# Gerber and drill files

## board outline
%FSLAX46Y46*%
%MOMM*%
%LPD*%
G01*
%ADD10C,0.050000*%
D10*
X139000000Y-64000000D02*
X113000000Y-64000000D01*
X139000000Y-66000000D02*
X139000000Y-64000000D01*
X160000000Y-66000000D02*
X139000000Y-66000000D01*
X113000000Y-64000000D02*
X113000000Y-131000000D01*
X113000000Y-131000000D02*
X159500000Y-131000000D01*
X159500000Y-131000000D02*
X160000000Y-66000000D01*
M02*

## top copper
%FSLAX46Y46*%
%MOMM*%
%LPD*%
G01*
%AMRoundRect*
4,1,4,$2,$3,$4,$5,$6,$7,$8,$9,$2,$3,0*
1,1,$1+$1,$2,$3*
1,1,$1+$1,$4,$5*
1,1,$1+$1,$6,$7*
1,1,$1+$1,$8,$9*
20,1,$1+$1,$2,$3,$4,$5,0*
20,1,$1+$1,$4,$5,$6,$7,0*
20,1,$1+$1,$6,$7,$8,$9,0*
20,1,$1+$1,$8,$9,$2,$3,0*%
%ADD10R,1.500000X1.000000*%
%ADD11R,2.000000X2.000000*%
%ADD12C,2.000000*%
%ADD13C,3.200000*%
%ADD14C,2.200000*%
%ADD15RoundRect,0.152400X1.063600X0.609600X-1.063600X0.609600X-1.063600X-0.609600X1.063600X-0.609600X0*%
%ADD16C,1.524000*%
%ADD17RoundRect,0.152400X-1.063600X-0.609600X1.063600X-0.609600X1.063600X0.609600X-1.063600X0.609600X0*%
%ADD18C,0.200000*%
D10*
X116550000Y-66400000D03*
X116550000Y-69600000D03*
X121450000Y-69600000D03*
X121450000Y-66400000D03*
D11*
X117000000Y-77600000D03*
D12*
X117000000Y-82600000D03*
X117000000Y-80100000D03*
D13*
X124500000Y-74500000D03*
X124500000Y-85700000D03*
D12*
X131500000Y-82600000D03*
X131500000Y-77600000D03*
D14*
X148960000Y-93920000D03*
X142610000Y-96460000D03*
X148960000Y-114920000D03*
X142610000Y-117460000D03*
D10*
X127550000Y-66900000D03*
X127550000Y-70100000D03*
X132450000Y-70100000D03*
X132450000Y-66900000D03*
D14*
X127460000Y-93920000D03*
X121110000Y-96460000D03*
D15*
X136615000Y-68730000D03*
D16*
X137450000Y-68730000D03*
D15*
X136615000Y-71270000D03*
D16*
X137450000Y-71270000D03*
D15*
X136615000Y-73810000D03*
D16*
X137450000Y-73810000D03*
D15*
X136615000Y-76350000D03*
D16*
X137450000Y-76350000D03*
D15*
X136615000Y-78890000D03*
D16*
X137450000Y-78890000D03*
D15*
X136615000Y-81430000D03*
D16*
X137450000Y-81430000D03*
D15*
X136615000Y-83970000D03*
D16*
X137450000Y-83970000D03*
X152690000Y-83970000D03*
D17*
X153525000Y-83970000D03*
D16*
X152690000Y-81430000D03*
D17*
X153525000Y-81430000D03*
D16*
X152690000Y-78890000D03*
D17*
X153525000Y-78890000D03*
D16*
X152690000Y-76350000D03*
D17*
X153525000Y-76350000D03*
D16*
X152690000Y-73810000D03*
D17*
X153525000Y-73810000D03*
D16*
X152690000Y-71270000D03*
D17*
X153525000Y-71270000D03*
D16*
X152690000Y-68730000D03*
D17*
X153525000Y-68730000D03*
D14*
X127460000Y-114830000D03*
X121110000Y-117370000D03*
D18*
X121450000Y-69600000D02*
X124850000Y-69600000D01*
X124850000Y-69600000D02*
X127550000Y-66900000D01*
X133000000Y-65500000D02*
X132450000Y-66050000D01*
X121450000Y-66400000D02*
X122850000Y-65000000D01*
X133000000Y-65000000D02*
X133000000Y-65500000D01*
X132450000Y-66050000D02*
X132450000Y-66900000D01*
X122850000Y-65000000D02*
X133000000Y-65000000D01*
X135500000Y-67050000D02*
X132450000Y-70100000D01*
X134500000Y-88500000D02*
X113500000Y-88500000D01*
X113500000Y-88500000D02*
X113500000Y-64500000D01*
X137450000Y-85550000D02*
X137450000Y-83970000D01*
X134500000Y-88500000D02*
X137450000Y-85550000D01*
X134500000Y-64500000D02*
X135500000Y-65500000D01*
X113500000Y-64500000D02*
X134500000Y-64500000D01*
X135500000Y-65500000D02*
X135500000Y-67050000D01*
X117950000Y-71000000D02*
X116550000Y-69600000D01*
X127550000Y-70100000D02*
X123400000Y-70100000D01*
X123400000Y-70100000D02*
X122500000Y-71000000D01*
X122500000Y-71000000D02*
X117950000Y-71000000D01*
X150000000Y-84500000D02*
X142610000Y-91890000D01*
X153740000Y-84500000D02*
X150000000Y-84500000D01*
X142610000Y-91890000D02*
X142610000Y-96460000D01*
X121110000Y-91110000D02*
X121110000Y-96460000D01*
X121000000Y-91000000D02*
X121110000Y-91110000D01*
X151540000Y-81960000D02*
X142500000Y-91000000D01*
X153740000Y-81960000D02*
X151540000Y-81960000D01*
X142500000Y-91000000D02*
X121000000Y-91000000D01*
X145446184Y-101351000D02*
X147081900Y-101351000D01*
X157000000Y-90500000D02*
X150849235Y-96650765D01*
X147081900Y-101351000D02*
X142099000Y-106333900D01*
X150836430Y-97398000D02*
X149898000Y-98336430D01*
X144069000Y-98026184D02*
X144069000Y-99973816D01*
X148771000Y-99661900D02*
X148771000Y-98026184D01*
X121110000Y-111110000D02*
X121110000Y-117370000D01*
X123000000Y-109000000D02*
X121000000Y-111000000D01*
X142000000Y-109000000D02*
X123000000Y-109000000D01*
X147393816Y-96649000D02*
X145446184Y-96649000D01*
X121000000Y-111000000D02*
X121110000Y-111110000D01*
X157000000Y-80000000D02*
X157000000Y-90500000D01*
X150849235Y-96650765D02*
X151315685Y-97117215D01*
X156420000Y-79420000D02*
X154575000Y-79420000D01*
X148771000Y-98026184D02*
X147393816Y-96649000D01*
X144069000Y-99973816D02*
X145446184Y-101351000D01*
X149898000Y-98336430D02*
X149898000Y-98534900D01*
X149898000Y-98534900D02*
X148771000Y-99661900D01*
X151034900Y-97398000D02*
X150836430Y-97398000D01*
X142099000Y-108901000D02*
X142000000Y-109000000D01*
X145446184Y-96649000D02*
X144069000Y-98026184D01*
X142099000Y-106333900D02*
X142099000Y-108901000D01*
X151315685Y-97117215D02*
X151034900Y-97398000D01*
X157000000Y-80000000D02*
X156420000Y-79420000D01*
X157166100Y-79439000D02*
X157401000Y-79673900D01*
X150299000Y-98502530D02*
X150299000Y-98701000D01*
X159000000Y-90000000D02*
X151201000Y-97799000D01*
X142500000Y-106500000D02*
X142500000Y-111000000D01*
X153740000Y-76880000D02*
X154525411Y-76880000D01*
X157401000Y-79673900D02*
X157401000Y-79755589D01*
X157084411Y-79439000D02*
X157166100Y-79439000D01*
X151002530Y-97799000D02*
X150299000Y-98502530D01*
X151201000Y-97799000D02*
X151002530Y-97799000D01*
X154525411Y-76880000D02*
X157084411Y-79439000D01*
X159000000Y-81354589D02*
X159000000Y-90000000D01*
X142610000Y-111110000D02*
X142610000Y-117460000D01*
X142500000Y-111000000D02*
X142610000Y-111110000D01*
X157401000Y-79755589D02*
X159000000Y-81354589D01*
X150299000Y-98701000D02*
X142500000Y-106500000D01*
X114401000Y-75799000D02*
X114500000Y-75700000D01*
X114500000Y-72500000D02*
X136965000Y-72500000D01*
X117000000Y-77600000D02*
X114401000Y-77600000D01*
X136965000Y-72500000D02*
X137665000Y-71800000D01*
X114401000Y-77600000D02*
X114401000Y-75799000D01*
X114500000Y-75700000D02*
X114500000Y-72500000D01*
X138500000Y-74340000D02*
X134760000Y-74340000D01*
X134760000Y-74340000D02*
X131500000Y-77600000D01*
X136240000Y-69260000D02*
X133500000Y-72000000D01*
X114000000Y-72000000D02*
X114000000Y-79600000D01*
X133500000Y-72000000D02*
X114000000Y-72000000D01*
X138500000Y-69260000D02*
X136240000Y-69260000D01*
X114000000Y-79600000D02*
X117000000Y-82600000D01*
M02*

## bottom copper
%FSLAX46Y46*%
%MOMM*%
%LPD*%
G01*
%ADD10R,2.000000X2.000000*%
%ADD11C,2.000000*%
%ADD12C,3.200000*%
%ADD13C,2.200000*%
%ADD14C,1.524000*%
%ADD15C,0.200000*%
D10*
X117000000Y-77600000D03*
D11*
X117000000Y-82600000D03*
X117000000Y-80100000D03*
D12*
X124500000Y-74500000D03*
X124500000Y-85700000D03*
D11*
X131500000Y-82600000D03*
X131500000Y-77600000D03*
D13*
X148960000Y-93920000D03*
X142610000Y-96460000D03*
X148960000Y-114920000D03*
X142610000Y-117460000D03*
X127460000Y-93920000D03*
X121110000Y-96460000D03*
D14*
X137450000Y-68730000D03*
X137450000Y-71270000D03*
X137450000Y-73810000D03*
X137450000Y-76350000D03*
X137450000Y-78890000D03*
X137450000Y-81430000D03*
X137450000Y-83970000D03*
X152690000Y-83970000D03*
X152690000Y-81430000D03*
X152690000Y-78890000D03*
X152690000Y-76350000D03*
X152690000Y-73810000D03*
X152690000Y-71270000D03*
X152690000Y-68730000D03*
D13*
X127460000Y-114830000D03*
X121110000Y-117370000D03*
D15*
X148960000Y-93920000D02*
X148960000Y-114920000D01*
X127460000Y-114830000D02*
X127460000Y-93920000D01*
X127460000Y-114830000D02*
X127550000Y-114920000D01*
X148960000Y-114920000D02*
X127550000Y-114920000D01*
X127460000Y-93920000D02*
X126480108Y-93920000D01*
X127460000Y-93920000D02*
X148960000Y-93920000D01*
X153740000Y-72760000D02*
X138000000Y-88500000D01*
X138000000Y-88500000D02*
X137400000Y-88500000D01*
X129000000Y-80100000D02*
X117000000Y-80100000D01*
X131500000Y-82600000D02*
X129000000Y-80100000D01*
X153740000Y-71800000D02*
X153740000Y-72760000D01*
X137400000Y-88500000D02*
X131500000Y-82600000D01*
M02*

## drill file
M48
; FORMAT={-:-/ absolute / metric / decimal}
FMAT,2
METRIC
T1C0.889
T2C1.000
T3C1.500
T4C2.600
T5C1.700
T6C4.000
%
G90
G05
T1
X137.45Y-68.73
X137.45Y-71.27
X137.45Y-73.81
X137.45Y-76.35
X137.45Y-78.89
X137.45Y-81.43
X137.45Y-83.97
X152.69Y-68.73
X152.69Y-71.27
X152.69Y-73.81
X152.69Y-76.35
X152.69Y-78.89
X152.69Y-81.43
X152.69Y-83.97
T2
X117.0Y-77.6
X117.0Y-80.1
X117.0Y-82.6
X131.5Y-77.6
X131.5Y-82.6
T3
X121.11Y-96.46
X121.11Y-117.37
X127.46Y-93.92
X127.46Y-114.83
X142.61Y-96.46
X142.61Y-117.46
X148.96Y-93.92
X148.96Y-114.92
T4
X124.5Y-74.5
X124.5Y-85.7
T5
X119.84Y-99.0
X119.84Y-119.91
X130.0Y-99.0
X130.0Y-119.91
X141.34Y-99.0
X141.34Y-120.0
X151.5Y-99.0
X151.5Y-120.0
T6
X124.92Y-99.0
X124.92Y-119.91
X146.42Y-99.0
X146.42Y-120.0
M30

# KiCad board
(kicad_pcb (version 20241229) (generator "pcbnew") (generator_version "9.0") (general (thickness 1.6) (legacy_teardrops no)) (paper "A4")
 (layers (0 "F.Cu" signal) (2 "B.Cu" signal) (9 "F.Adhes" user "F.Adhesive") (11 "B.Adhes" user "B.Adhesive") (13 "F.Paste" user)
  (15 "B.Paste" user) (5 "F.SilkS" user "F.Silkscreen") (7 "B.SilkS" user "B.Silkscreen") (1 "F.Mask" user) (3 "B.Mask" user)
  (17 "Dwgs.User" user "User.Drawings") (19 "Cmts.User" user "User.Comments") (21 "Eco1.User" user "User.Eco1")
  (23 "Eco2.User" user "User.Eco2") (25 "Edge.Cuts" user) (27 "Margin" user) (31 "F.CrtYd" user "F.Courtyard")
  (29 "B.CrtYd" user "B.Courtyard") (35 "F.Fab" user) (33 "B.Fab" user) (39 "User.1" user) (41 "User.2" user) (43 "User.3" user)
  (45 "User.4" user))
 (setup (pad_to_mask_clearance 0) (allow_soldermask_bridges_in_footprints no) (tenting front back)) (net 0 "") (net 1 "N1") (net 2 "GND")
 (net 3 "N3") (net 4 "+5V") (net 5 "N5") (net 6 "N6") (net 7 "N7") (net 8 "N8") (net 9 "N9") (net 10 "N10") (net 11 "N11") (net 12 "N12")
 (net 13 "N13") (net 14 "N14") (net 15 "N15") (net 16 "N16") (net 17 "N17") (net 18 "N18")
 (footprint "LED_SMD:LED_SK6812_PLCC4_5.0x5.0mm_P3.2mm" (layer "F.Cu") (at 119 68)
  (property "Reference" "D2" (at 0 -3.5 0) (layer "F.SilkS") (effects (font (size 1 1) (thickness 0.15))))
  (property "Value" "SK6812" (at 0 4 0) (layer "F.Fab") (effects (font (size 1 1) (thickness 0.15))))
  (pad "1" smd rect (at -2.45 -1.6 180) (size 1.5 1) (layers "F.Cu" "F.Mask" "F.Paste") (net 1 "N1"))
  (pad "2" smd rect (at -2.45 1.6 180) (size 1.5 1) (layers "F.Cu" "F.Mask" "F.Paste") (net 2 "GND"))
  (pad "3" smd rect (at 2.45 1.6 180) (size 1.5 1) (layers "F.Cu" "F.Mask" "F.Paste") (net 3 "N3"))
  (pad "4" smd rect (at 2.45 -1.6 180) (size 1.5 1) (layers "F.Cu" "F.Mask" "F.Paste") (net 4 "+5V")))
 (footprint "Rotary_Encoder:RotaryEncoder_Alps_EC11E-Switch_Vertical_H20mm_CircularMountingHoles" (layer "F.Cu") (at 117 77.6)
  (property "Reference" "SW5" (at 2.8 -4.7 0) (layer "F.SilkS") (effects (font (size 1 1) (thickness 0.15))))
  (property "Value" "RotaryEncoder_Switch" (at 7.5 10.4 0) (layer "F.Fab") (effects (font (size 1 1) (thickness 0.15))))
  (pad "A" thru_hole rect (at 0 0) (size 2 2) (drill 1) (layers "*.Cu" "*.Mask") (remove_unused_layers no) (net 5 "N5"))
  (pad "B" thru_hole circle (at 0 5) (size 2 2) (drill 1) (layers "*.Cu" "*.Mask") (remove_unused_layers no) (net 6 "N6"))
  (pad "C" thru_hole circle (at 0 2.5) (size 2 2) (drill 1) (layers "*.Cu" "*.Mask") (remove_unused_layers no) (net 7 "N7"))
  (pad "MP" thru_hole circle (at 7.5 -3.1) (size 3.2 3.2) (drill 2.6) (layers "*.Cu" "*.Mask") (remove_unused_layers no))
  (pad "MP" thru_hole circle (at 7.5 8.1) (size 3.2 3.2) (drill 2.6) (layers "*.Cu" "*.Mask") (remove_unused_layers no))
  (pad "S1" thru_hole circle (at 14.5 5) (size 2 2) (drill 1) (layers "*.Cu" "*.Mask") (remove_unused_layers no) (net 7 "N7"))
  (pad "S2" thru_hole circle (at 14.5 0) (size 2 2) (drill 1) (layers "*.Cu" "*.Mask") (remove_unused_layers no) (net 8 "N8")))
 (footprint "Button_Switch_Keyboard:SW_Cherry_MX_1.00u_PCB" (layer "F.Cu") (at 148.96 93.92)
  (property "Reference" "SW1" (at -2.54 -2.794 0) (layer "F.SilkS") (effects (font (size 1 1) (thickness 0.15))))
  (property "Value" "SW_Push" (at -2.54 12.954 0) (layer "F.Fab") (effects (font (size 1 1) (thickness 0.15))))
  (pad "" np_thru_hole circle (at -7.62 5.08) (size 1.7 1.7) (drill 1.7) (layers "*.Cu" "*.Mask"))
  (pad "" np_thru_hole circle (at -2.54 5.08) (size 4 4) (drill 4) (layers "*.Cu" "*.Mask"))
  (pad "" np_thru_hole circle (at 2.54 5.08) (size 1.7 1.7) (drill 1.7) (layers "*.Cu" "*.Mask"))
  (pad "1" thru_hole circle (at 0 0) (size 2.2 2.2) (drill 1.5) (layers "*.Cu" "*.Mask") (remove_unused_layers no) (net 2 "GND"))
  (pad "2" thru_hole circle (at -6.35 2.54) (size 2.2 2.2) (drill 1.5) (layers "*.Cu" "*.Mask") (remove_unused_layers no) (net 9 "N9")))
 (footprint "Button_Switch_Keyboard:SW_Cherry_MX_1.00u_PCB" (layer "F.Cu") (at 148.96 114.92)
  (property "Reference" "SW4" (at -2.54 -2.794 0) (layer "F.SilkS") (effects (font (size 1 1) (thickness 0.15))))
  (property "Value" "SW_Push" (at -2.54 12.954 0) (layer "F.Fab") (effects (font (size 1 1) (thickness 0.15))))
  (pad "" np_thru_hole circle (at -7.62 5.08) (size 1.7 1.7) (drill 1.7) (layers "*.Cu" "*.Mask"))
  (pad "" np_thru_hole circle (at -2.54 5.08) (size 4 4) (drill 4) (layers "*.Cu" "*.Mask"))
  (pad "" np_thru_hole circle (at 2.54 5.08) (size 1.7 1.7) (drill 1.7) (layers "*.Cu" "*.Mask"))
  (pad "1" thru_hole circle (at 0 0) (size 2.2 2.2) (drill 1.5) (layers "*.Cu" "*.Mask") (remove_unused_layers no) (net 2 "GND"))
  (pad "2" thru_hole circle (at -6.35 2.54) (size 2.2 2.2) (drill 1.5) (layers "*.Cu" "*.Mask") (remove_unused_layers no) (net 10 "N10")))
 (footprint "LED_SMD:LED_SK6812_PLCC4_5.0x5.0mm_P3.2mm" (layer "F.Cu") (at 130 68.5)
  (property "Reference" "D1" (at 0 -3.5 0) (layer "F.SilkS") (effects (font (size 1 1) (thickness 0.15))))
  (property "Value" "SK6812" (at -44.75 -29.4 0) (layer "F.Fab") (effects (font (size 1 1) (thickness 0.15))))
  (pad "1" smd rect (at -2.45 -1.6 180) (size 1.5 1) (layers "F.Cu" "F.Mask" "F.Paste") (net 3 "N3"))
  (pad "2" smd rect (at -2.45 1.6 180) (size 1.5 1) (layers "F.Cu" "F.Mask" "F.Paste") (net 2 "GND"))
  (pad "3" smd rect (at 2.45 1.6 180) (size 1.5 1) (layers "F.Cu" "F.Mask" "F.Paste") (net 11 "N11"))
  (pad "4" smd rect (at 2.45 -1.6 180) (size 1.5 1) (layers "F.Cu" "F.Mask" "F.Paste") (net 4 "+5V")))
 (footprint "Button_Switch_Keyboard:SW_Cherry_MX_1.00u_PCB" (layer "F.Cu") (at 127.46 93.92)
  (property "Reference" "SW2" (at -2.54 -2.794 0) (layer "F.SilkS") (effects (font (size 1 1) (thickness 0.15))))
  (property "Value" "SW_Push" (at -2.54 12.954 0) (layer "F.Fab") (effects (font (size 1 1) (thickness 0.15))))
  (pad "" np_thru_hole circle (at -7.62 5.08) (size 1.7 1.7) (drill 1.7) (layers "*.Cu" "*.Mask"))
  (pad "" np_thru_hole circle (at -2.54 5.08) (size 4 4) (drill 4) (layers "*.Cu" "*.Mask"))
  (pad "" np_thru_hole circle (at 2.54 5.08) (size 1.7 1.7) (drill 1.7) (layers "*.Cu" "*.Mask"))
  (pad "1" thru_hole circle (at 0 0) (size 2.2 2.2) (drill 1.5) (layers "*.Cu" "*.Mask") (remove_unused_layers no) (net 2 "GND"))
  (pad "2" thru_hole circle (at -6.35 2.54) (size 2.2 2.2) (drill 1.5) (layers "*.Cu" "*.Mask") (remove_unused_layers no) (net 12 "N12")))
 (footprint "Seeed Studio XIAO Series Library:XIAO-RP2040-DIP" (layer "F.Cu") (at 145.07 76.35)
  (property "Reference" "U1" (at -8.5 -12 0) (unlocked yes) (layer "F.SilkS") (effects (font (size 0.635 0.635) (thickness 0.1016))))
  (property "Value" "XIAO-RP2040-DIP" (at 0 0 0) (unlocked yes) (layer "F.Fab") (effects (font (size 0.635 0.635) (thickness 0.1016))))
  (pad "1" smd roundrect (at -8.455 -7.62 180) (size 2.432 1.524) (layers "F.Cu" "F.Mask") (roundrect_rratio 0.1) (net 6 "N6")
   (thermal_bridge_angle 45))
  (pad "1" thru_hole circle (at -7.62 -7.62 180) (size 1.524 1.524) (drill 0.889) (layers "*.Cu" "*.Mask") (remove_unused_layers no)
   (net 6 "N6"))
  (pad "2" smd roundrect (at -8.455 -5.08 180) (size 2.432 1.524) (layers "F.Cu" "F.Mask") (roundrect_rratio 0.1) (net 5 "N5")
   (thermal_bridge_angle 45))
  (pad "2" thru_hole circle (at -7.62 -5.08 180) (size 1.524 1.524) (drill 0.889) (layers "*.Cu" "*.Mask") (remove_unused_layers no)
   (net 5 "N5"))
  (pad "3" smd roundrect (at -8.455 -2.54 180) (size 2.432 1.524) (layers "F.Cu" "F.Mask") (roundrect_rratio 0.1) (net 8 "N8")
   (thermal_bridge_angle 45))
  (pad "3" thru_hole circle (at -7.62 -2.54 180) (size 1.524 1.524) (drill 0.889) (layers "*.Cu" "*.Mask") (remove_unused_layers no)
   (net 8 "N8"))
  (pad "4" smd roundrect (at -8.455 0 180) (size 2.432 1.524) (layers "F.Cu" "F.Mask") (roundrect_rratio 0.1) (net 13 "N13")
   (thermal_bridge_angle 45))
  (pad "4" thru_hole circle (at -7.62 0 180) (size 1.524 1.524) (drill 0.889) (layers "*.Cu" "*.Mask") (remove_unused_layers no)
   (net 13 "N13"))
  (pad "5" smd roundrect (at -8.455 2.54 180) (size 2.432 1.524) (layers "F.Cu" "F.Mask") (roundrect_rratio 0.1) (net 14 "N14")
   (thermal_bridge_angle 45))
  (pad "5" thru_hole circle (at -7.62 2.54 180) (size 1.524 1.524) (drill 0.889) (layers "*.Cu" "*.Mask") (remove_unused_layers no)
   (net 14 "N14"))
  (pad "6" smd roundrect (at -8.455 5.08 180) (size 2.432 1.524) (layers "F.Cu" "F.Mask") (roundrect_rratio 0.1) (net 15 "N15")
   (thermal_bridge_angle 45))
  (pad "6" thru_hole circle (at -7.62 5.08 180) (size 1.524 1.524) (drill 0.889) (layers "*.Cu" "*.Mask") (remove_unused_layers no)
   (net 15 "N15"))
  (pad "7" smd roundrect (at -8.455 7.62 180) (size 2.432 1.524) (layers "F.Cu" "F.Mask") (roundrect_rratio 0.1) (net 11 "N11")
   (thermal_bridge_angle 45))
  (pad "7" thru_hole circle (at -7.62 7.62 180) (size 1.524 1.524) (drill 0.889) (layers "*.Cu" "*.Mask") (remove_unused_layers no)
   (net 11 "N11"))
  (pad "8" thru_hole circle (at 7.62 7.62) (size 1.524 1.524) (drill 0.889) (layers "*.Cu" "*.Mask") (remove_unused_layers no) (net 9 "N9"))
  (pad "8" smd roundrect (at 8.455 7.62) (size 2.432 1.524) (layers "F.Cu" "F.Mask") (roundrect_rratio 0.1) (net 9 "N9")
   (thermal_bridge_angle 45))
  (pad "9" thru_hole circle (at 7.62 5.08) (size 1.524 1.524) (drill 0.889) (layers "*.Cu" "*.Mask") (remove_unused_layers no)
   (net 12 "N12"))
  (pad "9" smd roundrect (at 8.455 5.08) (size 2.432 1.524) (layers "F.Cu" "F.Mask") (roundrect_rratio 0.1) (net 12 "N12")
   (thermal_bridge_angle 45))
  (pad "10" thru_hole circle (at 7.62 2.54) (size 1.524 1.524) (drill 0.889) (layers "*.Cu" "*.Mask") (remove_unused_layers no)
   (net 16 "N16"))
  (pad "10" smd roundrect (at 8.455 2.54) (size 2.432 1.524) (layers "F.Cu" "F.Mask") (roundrect_rratio 0.1) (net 16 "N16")
   (thermal_bridge_angle 45))
  (pad "11" thru_hole circle (at 7.62 0) (size 1.524 1.524) (drill 0.889) (layers "*.Cu" "*.Mask") (remove_unused_layers no) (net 10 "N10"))
  (pad "11" smd roundrect (at 8.455 0) (size 2.432 1.524) (layers "F.Cu" "F.Mask") (roundrect_rratio 0.1) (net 10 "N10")
   (thermal_bridge_angle 45))
  (pad "12" thru_hole circle (at 7.62 -2.54) (size 1.524 1.524) (drill 0.889) (layers "*.Cu" "*.Mask") (remove_unused_layers no)
   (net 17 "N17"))
  (pad "12" smd roundrect (at 8.455 -2.54) (size 2.432 1.524) (layers "F.Cu" "F.Mask") (roundrect_rratio 0.1) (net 17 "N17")
   (thermal_bridge_angle 45))
  (pad "13" thru_hole circle (at 7.62 -5.08) (size 1.524 1.524) (drill 0.889) (layers "*.Cu" "*.Mask") (remove_unused_layers no)
   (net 7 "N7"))
  (pad "13" smd roundrect (at 8.455 -5.08) (size 2.432 1.524) (layers "F.Cu" "F.Mask") (roundrect_rratio 0.1) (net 7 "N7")
   (thermal_bridge_angle 45))
  (pad "14" thru_hole circle (at 7.62 -7.62) (size 1.524 1.524) (drill 0.889) (layers "*.Cu" "*.Mask") (remove_unused_layers no)
   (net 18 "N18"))
  (pad "14" smd roundrect (at 8.455 -7.62) (size 2.432 1.524) (layers "F.Cu" "F.Mask") (roundrect_rratio 0.1) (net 18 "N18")
   (thermal_bridge_angle 45)))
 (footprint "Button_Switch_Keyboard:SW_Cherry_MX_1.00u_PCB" (layer "F.Cu") (at 127.46 114.83)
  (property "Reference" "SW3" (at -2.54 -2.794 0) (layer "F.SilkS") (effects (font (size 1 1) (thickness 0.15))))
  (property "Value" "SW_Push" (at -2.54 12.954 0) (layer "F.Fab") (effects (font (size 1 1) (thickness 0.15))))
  (pad "" np_thru_hole circle (at -7.62 5.08) (size 1.7 1.7) (drill 1.7) (layers "*.Cu" "*.Mask"))
  (pad "" np_thru_hole circle (at -2.54 5.08) (size 4 4) (drill 4) (layers "*.Cu" "*.Mask"))
  (pad "" np_thru_hole circle (at 2.54 5.08) (size 1.7 1.7) (drill 1.7) (layers "*.Cu" "*.Mask"))
  (pad "1" thru_hole circle (at 0 0) (size 2.2 2.2) (drill 1.5) (layers "*.Cu" "*.Mask") (remove_unused_layers no) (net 2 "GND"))
  (pad "2" thru_hole circle (at -6.35 2.54) (size 2.2 2.2) (drill 1.5) (layers "*.Cu" "*.Mask") (remove_unused_layers no) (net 16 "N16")))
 (gr_line (start 139 64) (end 113 64) (stroke (width 0.05) (type default)) (layer "Edge.Cuts"))
 (gr_line (start 139 66) (end 139 64) (stroke (width 0.05) (type default)) (layer "Edge.Cuts"))
 (gr_line (start 160 66) (end 139 66) (stroke (width 0.05) (type default)) (locked yes) (layer "Edge.Cuts"))
 (gr_line (start 113 64) (end 113 131) (stroke (width 0.05) (type default)) (layer "Edge.Cuts"))
 (gr_line (start 113 131) (end 159.5 131) (stroke (width 0.05) (type default)) (layer "Edge.Cuts"))
 (gr_line (start 159.5 131) (end 160 66) (stroke (width 0.05) (type default)) (layer "Edge.Cuts"))
 (segment (start 121.45 69.6) (end 124.85 69.6) (width 0.2) (layer "F.Cu") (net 3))
 (segment (start 124.85 69.6) (end 127.55 66.9) (width 0.2) (layer "F.Cu") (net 3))
 (segment (start 133 65.5) (end 132.45 66.05) (width 0.2) (layer "F.Cu") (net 4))
 (segment (start 121.45 66.4) (end 122.85 65) (width 0.2) (layer "F.Cu") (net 4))
 (segment (start 133 65) (end 133 65.5) (width 0.2) (layer "F.Cu") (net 4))
 (segment (start 132.45 66.05) (end 132.45 66.9) (width 0.2) (layer "F.Cu") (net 4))
 (segment (start 122.85 65) (end 133 65) (width 0.2) (layer "F.Cu") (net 4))
 (segment (start 135.5 67.05) (end 132.45 70.1) (width 0.2) (layer "F.Cu") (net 11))
 (segment (start 134.5 88.5) (end 113.5 88.5) (width 0.2) (layer "F.Cu") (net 11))
 (segment (start 113.5 88.5) (end 113.5 64.5) (width 0.2) (layer "F.Cu") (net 11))
 (segment (start 137.45 85.55) (end 137.45 83.97) (width 0.2) (layer "F.Cu") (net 11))
 (segment (start 134.5 88.5) (end 137.45 85.55) (width 0.2) (layer "F.Cu") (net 11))
 (segment (start 134.5 64.5) (end 135.5 65.5) (width 0.2) (layer "F.Cu") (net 11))
 (segment (start 113.5 64.5) (end 134.5 64.5) (width 0.2) (layer "F.Cu") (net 11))
 (segment (start 135.5 65.5) (end 135.5 67.05) (width 0.2) (layer "F.Cu") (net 11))
 (segment (start 117.95 71) (end 116.55 69.6) (width 0.2) (layer "F.Cu") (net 2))
 (segment (start 127.55 70.1) (end 123.4 70.1) (width 0.2) (layer "F.Cu") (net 2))
 (segment (start 123.4 70.1) (end 122.5 71) (width 0.2) (layer "F.Cu") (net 2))
 (segment (start 122.5 71) (end 117.95 71) (width 0.2) (layer "F.Cu") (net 2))
 (segment (start 148.96 93.92) (end 148.96 114.92) (width 0.2) (layer "B.Cu") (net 2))
 (segment (start 127.46 114.83) (end 127.46 93.92) (width 0.2) (layer "B.Cu") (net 2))
 (segment (start 127.46 114.83) (end 127.55 114.92) (width 0.2) (layer "B.Cu") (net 2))
 (segment (start 148.96 114.92) (end 127.55 114.92) (width 0.2) (layer "B.Cu") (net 2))
 (segment (start 127.46 93.92) (end 126.480108 93.92) (width 0.2) (layer "B.Cu") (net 2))
 (segment (start 127.46 93.92) (end 148.96 93.92) (width 0.2) (layer "B.Cu") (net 2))
 (segment (start 150 84.5) (end 142.61 91.89) (width 0.2) (layer "F.Cu") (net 9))
 (segment (start 153.74 84.5) (end 150 84.5) (width 0.2) (layer "F.Cu") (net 9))
 (segment (start 142.61 91.89) (end 142.61 96.46) (width 0.2) (layer "F.Cu") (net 9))
 (segment (start 121.11 91.11) (end 121.11 96.46) (width 0.2) (layer "F.Cu") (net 12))
 (segment (start 121 91) (end 121.11 91.11) (width 0.2) (layer "F.Cu") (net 12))
 (segment (start 151.54 81.96) (end 142.5 91) (width 0.2) (layer "F.Cu") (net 12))
 (segment (start 153.74 81.96) (end 151.54 81.96) (width 0.2) (layer "F.Cu") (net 12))
 (segment (start 142.5 91) (end 121 91) (width 0.2) (layer "F.Cu") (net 12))
 (segment (start 145.446184 101.351) (end 147.0819 101.351) (width 0.2) (layer "F.Cu") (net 16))
 (segment (start 157 90.5) (end 150.849235 96.650765) (width 0.2) (layer "F.Cu") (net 16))
 (segment (start 147.0819 101.351) (end 142.099 106.3339) (width 0.2) (layer "F.Cu") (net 16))
 (segment (start 150.83643 97.398) (end 149.898 98.33643) (width 0.2) (layer "F.Cu") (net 16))
 (segment (start 144.069 98.026184) (end 144.069 99.973816) (width 0.2) (layer "F.Cu") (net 16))
 (segment (start 148.771 99.6619) (end 148.771 98.026184) (width 0.2) (layer "F.Cu") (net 16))
 (segment (start 121.11 111.11) (end 121.11 117.37) (width 0.2) (layer "F.Cu") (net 16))
 (segment (start 123 109) (end 121 111) (width 0.2) (layer "F.Cu") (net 16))
 (segment (start 142 109) (end 123 109) (width 0.2) (layer "F.Cu") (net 16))
 (segment (start 147.393816 96.649) (end 145.446184 96.649) (width 0.2) (layer "F.Cu") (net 16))
 (segment (start 121 111) (end 121.11 111.11) (width 0.2) (layer "F.Cu") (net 16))
 (segment (start 157 80) (end 157 90.5) (width 0.2) (layer "F.Cu") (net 16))
 (segment (start 150.849235 96.650765) (end 151.315685 97.117215) (width 0.2) (layer "F.Cu") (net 16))
 (segment (start 156.42 79.42) (end 154.575 79.42) (width 0.2) (layer "F.Cu") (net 16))
 (segment (start 148.771 98.026184) (end 147.393816 96.649) (width 0.2) (layer "F.Cu") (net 16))
 (segment (start 144.069 99.973816) (end 145.446184 101.351) (width 0.2) (layer "F.Cu") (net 16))
 (segment (start 149.898 98.33643) (end 149.898 98.5349) (width 0.2) (layer "F.Cu") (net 16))
 (segment (start 149.898 98.5349) (end 148.771 99.6619) (width 0.2) (layer "F.Cu") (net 16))
 (segment (start 151.0349 97.398) (end 150.83643 97.398) (width 0.2) (layer "F.Cu") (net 16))
 (segment (start 142.099 108.901) (end 142 109) (width 0.2) (layer "F.Cu") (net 16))
 (segment (start 145.446184 96.649) (end 144.069 98.026184) (width 0.2) (layer "F.Cu") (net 16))
 (segment (start 142.099 106.3339) (end 142.099 108.901) (width 0.2) (layer "F.Cu") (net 16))
 (segment (start 151.315685 97.117215) (end 151.0349 97.398) (width 0.2) (layer "F.Cu") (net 16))
 (segment (start 157 80) (end 156.42 79.42) (width 0.2) (layer "F.Cu") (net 16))
 (segment (start 157.1661 79.439) (end 157.401 79.6739) (width 0.2) (layer "F.Cu") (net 10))
 (segment (start 150.299 98.50253) (end 150.299 98.701) (width 0.2) (layer "F.Cu") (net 10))
 (segment (start 159 90) (end 151.201 97.799) (width 0.2) (layer "F.Cu") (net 10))
 (segment (start 142.5 106.5) (end 142.5 111) (width 0.2) (layer "F.Cu") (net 10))
 (segment (start 153.74 76.88) (end 154.525411 76.88) (width 0.2) (layer "F.Cu") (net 10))
 (segment (start 157.401 79.6739) (end 157.401 79.755589) (width 0.2) (layer "F.Cu") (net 10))
 (segment (start 157.084411 79.439) (end 157.1661 79.439) (width 0.2) (layer "F.Cu") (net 10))
 (segment (start 151.00253 97.799) (end 150.299 98.50253) (width 0.2) (layer "F.Cu") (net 10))
 (segment (start 151.201 97.799) (end 151.00253 97.799) (width 0.2) (layer "F.Cu") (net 10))
 (segment (start 154.525411 76.88) (end 157.084411 79.439) (width 0.2) (layer "F.Cu") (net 10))
 (segment (start 159 81.354589) (end 159 90) (width 0.2) (layer "F.Cu") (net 10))
 (segment (start 142.61 111.11) (end 142.61 117.46) (width 0.2) (layer "F.Cu") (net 10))
 (segment (start 142.5 111) (end 142.61 111.11) (width 0.2) (layer "F.Cu") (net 10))
 (segment (start 157.401 79.755589) (end 159 81.354589) (width 0.2) (layer "F.Cu") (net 10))
 (segment (start 150.299 98.701) (end 142.5 106.5) (width 0.2) (layer "F.Cu") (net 10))
 (segment (start 114.401 75.799) (end 114.5 75.7) (width 0.2) (layer "F.Cu") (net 5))
 (segment (start 114.5 72.5) (end 136.965 72.5) (width 0.2) (layer "F.Cu") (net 5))
 (segment (start 117 77.6) (end 114.401 77.6) (width 0.2) (layer "F.Cu") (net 5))
 (segment (start 136.965 72.5) (end 137.665 71.8) (width 0.2) (layer "F.Cu") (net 5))
 (segment (start 114.401 77.6) (end 114.401 75.799) (width 0.2) (layer "F.Cu") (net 5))
 (segment (start 114.5 75.7) (end 114.5 72.5) (width 0.2) (layer "F.Cu") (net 5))
 (segment (start 138.5 74.34) (end 134.76 74.34) (width 0.2) (layer "F.Cu") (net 8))
 (segment (start 134.76 74.34) (end 131.5 77.6) (width 0.2) (layer "F.Cu") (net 8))
 (segment (start 136.24 69.26) (end 133.5 72) (width 0.2) (layer "F.Cu") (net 6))
 (segment (start 114 72) (end 114 79.6) (width 0.2) (layer "F.Cu") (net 6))
 (segment (start 133.5 72) (end 114 72) (width 0.2) (layer "F.Cu") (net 6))
 (segment (start 138.5 69.26) (end 136.24 69.26) (width 0.2) (layer "F.Cu") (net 6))
 (segment (start 114 79.6) (end 117 82.6) (width 0.2) (layer "F.Cu") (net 6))
 (segment (start 153.74 72.76) (end 138 88.5) (width 0.2) (layer "B.Cu") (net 7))
 (segment (start 138 88.5) (end 137.4 88.5) (width 0.2) (layer "B.Cu") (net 7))
 (segment (start 129 80.1) (end 117 80.1) (width 0.2) (layer "B.Cu") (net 7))
 (segment (start 131.5 82.6) (end 129 80.1) (width 0.2) (layer "B.Cu") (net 7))
 (segment (start 153.74 71.8) (end 153.74 72.76) (width 0.2) (layer "B.Cu") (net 7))
 (segment (start 137.4 88.5) (end 131.5 82.6) (width 0.2) (layer "B.Cu") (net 7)))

